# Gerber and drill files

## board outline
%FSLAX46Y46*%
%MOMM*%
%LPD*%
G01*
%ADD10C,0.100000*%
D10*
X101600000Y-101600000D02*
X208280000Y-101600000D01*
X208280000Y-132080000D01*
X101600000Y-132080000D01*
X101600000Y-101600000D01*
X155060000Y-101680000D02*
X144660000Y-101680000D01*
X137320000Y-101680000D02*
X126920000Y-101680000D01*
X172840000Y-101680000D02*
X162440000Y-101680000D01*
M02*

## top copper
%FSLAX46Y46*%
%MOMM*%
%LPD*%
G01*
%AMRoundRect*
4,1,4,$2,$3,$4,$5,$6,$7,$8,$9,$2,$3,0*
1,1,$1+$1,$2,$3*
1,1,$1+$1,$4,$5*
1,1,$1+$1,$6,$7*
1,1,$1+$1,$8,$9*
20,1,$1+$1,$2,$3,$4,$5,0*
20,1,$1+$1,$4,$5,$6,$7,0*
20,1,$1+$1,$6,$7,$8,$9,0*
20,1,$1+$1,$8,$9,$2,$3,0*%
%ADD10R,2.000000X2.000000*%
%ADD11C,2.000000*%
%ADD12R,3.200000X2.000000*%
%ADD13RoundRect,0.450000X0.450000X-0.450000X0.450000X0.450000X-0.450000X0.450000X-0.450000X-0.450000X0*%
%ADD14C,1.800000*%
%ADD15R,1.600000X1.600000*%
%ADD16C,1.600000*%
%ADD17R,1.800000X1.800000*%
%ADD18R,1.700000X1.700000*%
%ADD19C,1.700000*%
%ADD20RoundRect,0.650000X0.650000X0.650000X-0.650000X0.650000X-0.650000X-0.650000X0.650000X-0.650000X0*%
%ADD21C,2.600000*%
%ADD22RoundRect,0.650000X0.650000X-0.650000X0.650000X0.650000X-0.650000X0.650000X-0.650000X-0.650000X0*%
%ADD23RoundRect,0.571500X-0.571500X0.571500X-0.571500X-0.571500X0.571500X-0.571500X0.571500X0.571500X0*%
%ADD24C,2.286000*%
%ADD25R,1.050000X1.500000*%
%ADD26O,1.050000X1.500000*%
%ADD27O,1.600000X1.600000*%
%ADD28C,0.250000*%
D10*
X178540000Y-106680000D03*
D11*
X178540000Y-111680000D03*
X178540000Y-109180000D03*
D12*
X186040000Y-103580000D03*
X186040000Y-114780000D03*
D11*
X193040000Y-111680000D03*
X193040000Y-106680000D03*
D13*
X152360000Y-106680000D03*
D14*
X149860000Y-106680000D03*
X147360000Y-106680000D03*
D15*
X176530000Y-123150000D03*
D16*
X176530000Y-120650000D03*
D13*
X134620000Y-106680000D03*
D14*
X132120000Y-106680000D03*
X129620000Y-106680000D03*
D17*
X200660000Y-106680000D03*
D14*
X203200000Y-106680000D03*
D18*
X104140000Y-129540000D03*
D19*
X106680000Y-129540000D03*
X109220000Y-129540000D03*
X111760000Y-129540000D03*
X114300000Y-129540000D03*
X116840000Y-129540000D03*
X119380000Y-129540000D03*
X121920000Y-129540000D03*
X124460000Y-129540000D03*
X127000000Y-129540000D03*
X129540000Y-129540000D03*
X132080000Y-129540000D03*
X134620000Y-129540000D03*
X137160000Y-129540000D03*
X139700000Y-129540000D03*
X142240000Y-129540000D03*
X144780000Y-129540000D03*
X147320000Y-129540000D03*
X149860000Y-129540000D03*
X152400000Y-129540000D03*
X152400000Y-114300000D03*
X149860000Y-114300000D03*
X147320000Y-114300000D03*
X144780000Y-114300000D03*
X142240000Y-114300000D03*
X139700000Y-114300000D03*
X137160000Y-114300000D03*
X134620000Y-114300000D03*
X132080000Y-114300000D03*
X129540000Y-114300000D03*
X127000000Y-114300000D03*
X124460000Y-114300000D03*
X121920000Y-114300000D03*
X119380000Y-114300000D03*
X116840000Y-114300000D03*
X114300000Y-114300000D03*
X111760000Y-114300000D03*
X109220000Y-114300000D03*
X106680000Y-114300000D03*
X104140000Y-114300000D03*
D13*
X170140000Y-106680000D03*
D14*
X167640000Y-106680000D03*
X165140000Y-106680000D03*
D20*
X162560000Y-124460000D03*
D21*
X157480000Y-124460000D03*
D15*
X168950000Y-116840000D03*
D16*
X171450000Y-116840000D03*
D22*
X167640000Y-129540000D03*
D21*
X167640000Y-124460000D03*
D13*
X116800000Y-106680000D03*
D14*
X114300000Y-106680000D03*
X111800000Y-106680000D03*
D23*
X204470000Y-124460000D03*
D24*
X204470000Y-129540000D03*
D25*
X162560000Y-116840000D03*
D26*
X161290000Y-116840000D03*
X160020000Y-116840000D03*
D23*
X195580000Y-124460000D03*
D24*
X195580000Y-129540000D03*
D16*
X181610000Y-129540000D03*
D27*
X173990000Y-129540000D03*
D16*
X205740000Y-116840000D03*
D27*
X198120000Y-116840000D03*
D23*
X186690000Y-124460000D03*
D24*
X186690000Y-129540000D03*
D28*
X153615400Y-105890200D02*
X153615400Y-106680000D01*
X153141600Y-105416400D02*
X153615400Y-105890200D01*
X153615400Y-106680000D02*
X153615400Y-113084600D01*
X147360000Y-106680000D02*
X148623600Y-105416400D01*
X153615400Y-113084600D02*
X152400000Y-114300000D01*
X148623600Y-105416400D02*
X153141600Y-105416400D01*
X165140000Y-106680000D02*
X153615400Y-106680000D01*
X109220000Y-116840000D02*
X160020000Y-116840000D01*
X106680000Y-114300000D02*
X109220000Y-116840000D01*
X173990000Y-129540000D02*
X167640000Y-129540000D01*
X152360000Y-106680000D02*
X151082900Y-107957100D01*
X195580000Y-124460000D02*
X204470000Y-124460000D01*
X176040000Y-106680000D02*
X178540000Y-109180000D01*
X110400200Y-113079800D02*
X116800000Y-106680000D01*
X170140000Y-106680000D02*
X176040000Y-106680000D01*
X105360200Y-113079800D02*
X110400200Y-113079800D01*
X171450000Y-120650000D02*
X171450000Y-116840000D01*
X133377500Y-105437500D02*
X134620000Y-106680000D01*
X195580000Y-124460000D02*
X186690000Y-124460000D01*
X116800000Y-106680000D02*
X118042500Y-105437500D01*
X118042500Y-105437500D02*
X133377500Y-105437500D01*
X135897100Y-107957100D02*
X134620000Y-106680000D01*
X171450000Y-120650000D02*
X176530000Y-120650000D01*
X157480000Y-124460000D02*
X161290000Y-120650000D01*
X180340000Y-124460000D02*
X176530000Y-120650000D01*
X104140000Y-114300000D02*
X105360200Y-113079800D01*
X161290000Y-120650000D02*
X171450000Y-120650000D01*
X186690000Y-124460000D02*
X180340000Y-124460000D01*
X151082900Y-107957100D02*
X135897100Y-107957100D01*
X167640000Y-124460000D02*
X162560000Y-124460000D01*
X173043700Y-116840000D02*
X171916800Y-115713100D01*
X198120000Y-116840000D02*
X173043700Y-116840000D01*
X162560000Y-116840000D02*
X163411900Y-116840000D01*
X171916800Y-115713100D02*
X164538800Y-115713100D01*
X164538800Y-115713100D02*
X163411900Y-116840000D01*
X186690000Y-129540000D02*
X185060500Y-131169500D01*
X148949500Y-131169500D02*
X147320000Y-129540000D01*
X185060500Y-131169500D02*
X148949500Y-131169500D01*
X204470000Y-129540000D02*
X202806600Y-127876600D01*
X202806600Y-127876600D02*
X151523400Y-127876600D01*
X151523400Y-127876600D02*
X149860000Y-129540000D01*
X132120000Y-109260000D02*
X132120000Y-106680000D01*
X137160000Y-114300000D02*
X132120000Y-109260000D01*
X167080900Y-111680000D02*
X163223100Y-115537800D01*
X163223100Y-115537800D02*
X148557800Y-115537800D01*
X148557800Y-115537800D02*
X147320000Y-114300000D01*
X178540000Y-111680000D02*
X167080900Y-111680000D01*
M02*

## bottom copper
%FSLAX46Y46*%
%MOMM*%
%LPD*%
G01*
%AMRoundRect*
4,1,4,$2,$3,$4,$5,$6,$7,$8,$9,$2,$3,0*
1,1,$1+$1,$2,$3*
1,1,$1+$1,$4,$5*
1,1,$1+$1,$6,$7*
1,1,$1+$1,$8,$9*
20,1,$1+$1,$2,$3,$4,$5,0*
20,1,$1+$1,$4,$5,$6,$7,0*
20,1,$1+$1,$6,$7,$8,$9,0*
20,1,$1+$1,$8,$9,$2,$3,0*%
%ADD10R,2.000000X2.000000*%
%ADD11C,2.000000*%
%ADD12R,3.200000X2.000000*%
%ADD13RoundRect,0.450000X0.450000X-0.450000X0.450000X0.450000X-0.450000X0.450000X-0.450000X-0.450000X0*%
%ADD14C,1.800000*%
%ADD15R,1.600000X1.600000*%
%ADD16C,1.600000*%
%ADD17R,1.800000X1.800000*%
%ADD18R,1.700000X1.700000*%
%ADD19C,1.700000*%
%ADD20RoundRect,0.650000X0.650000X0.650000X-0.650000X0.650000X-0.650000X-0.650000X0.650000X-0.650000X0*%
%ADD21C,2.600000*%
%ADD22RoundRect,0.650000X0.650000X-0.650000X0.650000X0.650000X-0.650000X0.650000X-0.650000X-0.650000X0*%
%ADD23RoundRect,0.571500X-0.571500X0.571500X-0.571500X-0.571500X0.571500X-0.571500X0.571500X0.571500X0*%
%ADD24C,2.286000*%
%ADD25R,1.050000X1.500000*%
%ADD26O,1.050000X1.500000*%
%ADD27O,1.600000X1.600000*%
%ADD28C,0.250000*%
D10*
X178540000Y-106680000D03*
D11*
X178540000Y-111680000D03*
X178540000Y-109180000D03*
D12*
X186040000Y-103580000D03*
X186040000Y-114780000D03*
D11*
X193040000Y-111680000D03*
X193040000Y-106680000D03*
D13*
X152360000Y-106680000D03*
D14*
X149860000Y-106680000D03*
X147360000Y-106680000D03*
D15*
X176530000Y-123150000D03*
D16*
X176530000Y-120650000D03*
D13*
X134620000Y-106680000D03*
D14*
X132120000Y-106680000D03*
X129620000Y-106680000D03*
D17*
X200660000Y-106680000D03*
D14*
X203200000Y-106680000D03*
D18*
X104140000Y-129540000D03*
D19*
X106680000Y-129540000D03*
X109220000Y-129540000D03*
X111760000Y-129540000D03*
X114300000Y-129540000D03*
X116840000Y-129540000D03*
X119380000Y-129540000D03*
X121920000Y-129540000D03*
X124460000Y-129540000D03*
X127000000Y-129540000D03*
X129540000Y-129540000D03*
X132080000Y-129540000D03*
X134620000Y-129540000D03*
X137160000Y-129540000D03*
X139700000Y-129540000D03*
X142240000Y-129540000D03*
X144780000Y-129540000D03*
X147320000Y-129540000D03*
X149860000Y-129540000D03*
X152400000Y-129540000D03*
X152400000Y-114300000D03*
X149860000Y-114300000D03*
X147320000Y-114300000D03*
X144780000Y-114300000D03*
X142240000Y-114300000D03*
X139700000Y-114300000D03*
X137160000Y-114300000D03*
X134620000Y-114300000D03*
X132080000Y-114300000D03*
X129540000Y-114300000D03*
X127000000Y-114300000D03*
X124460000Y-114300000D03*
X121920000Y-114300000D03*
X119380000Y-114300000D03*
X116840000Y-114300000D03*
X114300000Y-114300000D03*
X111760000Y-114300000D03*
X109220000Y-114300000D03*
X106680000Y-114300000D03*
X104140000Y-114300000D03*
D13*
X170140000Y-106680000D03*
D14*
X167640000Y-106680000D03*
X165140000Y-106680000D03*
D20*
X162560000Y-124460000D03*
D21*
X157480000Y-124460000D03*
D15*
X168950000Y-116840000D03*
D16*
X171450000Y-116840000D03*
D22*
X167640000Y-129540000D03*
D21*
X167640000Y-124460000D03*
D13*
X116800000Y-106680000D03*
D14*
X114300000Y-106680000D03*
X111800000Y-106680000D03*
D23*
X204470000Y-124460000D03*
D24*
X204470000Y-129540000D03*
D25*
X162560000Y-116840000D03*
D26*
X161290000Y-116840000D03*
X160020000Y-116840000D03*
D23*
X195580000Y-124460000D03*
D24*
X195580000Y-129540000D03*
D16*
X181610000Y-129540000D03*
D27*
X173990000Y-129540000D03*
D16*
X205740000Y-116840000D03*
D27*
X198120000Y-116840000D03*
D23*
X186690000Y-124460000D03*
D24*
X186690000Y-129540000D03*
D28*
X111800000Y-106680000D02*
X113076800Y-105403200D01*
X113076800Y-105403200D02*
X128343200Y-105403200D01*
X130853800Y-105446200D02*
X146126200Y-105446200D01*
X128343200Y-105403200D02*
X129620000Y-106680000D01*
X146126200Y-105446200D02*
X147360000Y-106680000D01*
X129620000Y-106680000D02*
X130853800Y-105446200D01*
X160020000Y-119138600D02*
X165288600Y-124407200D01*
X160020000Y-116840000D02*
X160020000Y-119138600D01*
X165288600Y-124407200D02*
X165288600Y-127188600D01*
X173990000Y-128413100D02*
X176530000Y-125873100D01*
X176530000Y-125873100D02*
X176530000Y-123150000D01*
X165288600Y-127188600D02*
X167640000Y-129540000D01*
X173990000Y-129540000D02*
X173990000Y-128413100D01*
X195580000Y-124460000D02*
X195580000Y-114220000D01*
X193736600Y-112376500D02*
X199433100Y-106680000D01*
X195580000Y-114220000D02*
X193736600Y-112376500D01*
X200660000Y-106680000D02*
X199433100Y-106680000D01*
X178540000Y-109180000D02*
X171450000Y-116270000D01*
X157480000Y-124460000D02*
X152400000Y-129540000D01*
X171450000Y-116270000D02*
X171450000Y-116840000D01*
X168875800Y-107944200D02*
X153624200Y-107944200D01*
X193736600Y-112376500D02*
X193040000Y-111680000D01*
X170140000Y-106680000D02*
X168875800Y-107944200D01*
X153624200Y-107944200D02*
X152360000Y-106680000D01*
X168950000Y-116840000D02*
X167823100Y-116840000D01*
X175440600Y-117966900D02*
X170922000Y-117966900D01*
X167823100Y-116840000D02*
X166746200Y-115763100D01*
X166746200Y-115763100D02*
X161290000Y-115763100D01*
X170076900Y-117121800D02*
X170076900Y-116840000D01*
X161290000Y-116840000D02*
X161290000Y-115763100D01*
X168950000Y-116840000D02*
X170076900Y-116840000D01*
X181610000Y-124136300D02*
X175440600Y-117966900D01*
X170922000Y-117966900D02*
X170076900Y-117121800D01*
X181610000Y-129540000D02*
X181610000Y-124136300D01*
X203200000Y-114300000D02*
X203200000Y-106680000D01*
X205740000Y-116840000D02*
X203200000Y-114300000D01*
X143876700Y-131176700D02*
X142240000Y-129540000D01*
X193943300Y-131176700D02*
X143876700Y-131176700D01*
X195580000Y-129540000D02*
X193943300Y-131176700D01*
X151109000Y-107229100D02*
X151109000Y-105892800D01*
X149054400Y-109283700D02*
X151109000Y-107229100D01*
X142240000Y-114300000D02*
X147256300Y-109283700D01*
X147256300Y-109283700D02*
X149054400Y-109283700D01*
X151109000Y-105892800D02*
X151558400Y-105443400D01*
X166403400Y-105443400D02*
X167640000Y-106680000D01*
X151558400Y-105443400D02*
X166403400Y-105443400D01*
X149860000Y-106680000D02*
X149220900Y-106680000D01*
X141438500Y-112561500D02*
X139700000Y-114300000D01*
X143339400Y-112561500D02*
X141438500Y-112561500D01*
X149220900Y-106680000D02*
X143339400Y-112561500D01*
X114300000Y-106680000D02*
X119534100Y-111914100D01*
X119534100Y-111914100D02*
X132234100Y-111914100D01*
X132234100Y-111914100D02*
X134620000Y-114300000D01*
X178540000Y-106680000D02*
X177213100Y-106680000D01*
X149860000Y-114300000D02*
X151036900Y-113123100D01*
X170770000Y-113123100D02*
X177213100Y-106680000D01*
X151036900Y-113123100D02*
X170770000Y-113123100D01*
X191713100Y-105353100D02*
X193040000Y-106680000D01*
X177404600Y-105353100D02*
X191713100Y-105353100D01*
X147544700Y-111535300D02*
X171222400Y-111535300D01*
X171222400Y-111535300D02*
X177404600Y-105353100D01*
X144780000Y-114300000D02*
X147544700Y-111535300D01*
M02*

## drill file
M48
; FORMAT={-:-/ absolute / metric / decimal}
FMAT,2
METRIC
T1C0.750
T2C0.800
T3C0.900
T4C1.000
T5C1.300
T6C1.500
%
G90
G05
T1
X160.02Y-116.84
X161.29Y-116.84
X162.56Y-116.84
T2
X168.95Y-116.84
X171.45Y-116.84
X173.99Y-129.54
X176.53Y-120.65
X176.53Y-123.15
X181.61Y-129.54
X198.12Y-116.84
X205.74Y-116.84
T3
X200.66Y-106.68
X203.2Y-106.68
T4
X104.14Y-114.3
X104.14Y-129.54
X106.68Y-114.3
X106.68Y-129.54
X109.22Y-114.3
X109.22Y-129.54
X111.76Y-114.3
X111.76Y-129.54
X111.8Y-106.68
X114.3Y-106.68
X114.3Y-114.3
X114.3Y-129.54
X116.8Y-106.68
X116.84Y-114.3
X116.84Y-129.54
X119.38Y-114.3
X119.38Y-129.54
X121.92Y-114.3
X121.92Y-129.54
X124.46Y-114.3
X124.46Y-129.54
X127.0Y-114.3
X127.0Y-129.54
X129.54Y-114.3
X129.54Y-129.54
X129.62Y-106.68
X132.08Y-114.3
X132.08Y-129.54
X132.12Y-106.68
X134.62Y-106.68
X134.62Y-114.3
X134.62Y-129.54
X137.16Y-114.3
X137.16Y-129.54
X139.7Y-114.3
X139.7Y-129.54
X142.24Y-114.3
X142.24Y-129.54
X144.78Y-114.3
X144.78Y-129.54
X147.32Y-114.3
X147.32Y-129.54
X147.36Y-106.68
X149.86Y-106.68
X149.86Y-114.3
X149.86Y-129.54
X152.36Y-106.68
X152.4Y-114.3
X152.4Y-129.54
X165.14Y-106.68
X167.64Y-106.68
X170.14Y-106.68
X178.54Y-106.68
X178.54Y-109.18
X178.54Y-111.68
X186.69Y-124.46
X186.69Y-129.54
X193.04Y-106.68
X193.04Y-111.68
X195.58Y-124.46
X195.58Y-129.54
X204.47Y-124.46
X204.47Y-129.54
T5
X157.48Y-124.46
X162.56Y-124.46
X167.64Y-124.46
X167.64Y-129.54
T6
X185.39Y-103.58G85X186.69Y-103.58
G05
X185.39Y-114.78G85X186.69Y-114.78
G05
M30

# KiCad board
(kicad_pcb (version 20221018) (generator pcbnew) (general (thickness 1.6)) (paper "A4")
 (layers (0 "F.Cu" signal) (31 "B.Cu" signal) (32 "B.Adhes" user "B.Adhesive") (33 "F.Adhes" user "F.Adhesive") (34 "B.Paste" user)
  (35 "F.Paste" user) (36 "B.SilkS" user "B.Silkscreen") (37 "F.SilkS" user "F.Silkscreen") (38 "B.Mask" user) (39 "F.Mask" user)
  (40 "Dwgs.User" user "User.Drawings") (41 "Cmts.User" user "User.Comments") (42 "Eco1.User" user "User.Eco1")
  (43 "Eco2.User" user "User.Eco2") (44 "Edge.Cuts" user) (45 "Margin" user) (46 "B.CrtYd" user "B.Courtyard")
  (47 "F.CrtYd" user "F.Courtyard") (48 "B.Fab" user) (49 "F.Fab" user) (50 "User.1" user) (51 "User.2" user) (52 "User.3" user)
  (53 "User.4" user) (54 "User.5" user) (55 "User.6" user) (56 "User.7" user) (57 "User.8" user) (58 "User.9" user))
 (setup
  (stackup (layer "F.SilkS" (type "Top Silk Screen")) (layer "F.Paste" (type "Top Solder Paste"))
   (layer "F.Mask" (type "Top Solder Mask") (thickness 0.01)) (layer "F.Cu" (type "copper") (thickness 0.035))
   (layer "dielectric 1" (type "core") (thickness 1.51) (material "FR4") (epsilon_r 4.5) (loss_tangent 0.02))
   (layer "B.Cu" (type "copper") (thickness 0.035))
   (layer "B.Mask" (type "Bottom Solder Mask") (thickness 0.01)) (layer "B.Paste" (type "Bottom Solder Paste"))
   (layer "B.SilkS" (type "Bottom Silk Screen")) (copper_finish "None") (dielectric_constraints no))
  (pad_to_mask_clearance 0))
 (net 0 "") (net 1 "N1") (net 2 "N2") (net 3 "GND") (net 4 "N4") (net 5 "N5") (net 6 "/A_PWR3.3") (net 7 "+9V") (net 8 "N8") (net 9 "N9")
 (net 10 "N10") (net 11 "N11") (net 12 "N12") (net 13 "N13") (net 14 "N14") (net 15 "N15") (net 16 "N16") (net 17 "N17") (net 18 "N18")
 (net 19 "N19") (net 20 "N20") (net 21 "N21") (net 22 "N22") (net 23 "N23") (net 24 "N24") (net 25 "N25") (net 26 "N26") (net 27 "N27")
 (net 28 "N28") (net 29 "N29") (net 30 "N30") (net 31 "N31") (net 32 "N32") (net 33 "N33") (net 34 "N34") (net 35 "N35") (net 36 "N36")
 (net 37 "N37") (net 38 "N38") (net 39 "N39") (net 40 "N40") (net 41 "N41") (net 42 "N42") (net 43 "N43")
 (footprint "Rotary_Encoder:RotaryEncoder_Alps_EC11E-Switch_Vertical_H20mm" (layer "F.Cu") (at 178.54 106.68)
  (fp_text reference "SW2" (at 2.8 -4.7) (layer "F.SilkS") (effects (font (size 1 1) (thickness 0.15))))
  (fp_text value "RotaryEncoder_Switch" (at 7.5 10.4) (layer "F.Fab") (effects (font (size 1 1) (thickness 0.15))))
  (pad "A" thru_hole rect (at 0 0) (size 2 2) (drill 1) (layers "*.Cu" "*.Mask") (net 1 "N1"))
  (pad "B" thru_hole circle (at 0 5) (size 2 2) (drill 1) (layers "*.Cu" "*.Mask") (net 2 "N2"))
  (pad "C" thru_hole circle (at 0 2.5) (size 2 2) (drill 1) (layers "*.Cu" "*.Mask") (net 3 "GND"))
  (pad "MP" thru_hole rect (at 7.5 -3.1) (size 3.2 2) (drill oval 2.8 1.5) (layers "*.Cu" "*.Mask"))
  (pad "MP" thru_hole rect (at 7.5 8.1) (size 3.2 2) (drill oval 2.8 1.5) (layers "*.Cu" "*.Mask"))
  (pad "S1" thru_hole circle (at 14.5 5) (size 2 2) (drill 1) (layers "*.Cu" "*.Mask") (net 3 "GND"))
  (pad "S2" thru_hole circle (at 14.5 0) (size 2 2) (drill 1) (layers "*.Cu" "*.Mask") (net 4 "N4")))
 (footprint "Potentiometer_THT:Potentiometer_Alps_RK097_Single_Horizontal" (layer "F.Cu") (at 152.36 106.68 -90)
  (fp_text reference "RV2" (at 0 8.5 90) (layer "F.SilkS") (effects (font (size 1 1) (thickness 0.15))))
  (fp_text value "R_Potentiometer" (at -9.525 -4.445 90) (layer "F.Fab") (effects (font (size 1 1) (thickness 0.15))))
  (fp_line (start -5 -2.7) (end -5 7.7) (stroke (width 0.1) (type solid)) (layer "Edge.Cuts"))
  (pad "1" thru_hole roundrect (at 0 0 90) (size 1.8 1.8) (drill 1) (layers "*.Cu" "*.Mask") (roundrect_rratio 0.25) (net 3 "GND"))
  (pad "2" thru_hole circle (at 0 2.5 90) (size 1.8 1.8) (drill 1) (layers "*.Cu" "*.Mask") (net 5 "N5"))
  (pad "3" thru_hole circle (at 0 5 90) (size 1.8 1.8) (drill 1) (layers "*.Cu" "*.Mask") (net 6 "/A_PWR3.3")))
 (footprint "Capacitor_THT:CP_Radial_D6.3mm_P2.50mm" (layer "F.Cu") (at 176.53 123.15 90)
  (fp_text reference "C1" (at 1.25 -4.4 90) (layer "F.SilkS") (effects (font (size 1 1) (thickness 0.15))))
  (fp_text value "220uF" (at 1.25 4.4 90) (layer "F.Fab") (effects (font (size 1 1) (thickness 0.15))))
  (pad "1" thru_hole rect (at 0 0 90) (size 1.6 1.6) (drill 0.8) (layers "*.Cu" "*.Mask") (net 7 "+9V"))
  (pad "2" thru_hole circle (at 2.5 0 90) (size 1.6 1.6) (drill 0.8) (layers "*.Cu" "*.Mask") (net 3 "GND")))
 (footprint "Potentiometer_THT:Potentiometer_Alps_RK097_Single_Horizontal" (layer "F.Cu") (at 134.62 106.68 -90)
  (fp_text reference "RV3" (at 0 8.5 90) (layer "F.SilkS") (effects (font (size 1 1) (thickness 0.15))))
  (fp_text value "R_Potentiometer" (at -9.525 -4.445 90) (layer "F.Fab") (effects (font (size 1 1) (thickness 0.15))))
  (fp_line (start -5 -2.7) (end -5 7.7) (stroke (width 0.1) (type solid)) (layer "Edge.Cuts"))
  (pad "1" thru_hole roundrect (at 0 0 90) (size 1.8 1.8) (drill 1) (layers "*.Cu" "*.Mask") (roundrect_rratio 0.25) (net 3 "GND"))
  (pad "2" thru_hole circle (at 0 2.5 90) (size 1.8 1.8) (drill 1) (layers "*.Cu" "*.Mask") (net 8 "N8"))
  (pad "3" thru_hole circle (at 0 5 90) (size 1.8 1.8) (drill 1) (layers "*.Cu" "*.Mask") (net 6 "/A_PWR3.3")))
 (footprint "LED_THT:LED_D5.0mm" (layer "F.Cu") (at 200.66 106.68)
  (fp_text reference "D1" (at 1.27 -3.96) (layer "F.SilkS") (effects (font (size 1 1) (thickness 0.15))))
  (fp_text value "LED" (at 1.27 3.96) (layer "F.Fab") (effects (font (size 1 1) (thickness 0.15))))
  (pad "1" thru_hole rect (at 0 0) (size 1.8 1.8) (drill 0.9) (layers "*.Cu" "*.Mask") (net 3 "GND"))
  (pad "2" thru_hole circle (at 2.54 0) (size 1.8 1.8) (drill 0.9) (layers "*.Cu" "*.Mask") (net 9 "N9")))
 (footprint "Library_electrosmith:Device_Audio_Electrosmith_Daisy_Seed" (layer "F.Cu") (at 104.14 129.54 90)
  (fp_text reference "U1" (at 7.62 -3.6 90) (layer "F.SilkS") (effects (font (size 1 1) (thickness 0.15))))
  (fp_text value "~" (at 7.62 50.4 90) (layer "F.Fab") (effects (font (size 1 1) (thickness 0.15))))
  (pad "1" thru_hole rect (at 0 0 90) (size 1.7 1.7) (drill 1) (layers "*.Cu" "*.Mask") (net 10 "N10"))
  (pad "2" thru_hole circle (at 0 2.54 90) (size 1.7 1.7) (drill 1) (layers "*.Cu" "*.Mask") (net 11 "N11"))
  (pad "3" thru_hole circle (at 0 5.08 90) (size 1.7 1.7) (drill 1) (layers "*.Cu" "*.Mask") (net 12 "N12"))
  (pad "4" thru_hole circle (at 0 7.62 90) (size 1.7 1.7) (drill 1) (layers "*.Cu" "*.Mask") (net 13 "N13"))
  (pad "5" thru_hole circle (at 0 10.16 90) (size 1.7 1.7) (drill 1) (layers "*.Cu" "*.Mask") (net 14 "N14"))
  (pad "6" thru_hole circle (at 0 12.7 90) (size 1.7 1.7) (drill 1) (layers "*.Cu" "*.Mask") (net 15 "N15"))
  (pad "7" thru_hole circle (at 0 15.24 90) (size 1.7 1.7) (drill 1) (layers "*.Cu" "*.Mask") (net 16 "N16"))
  (pad "8" thru_hole circle (at 0 17.78 90) (size 1.7 1.7) (drill 1) (layers "*.Cu" "*.Mask") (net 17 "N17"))
  (pad "9" thru_hole circle (at 0 20.32 90) (size 1.7 1.7) (drill 1) (layers "*.Cu" "*.Mask") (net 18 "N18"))
  (pad "10" thru_hole circle (at 0 22.86 90) (size 1.7 1.7) (drill 1) (layers "*.Cu" "*.Mask") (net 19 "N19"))
  (pad "11" thru_hole circle (at 0 25.4 90) (size 1.7 1.7) (drill 1) (layers "*.Cu" "*.Mask") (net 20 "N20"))
  (pad "12" thru_hole circle (at 0 27.94 90) (size 1.7 1.7) (drill 1) (layers "*.Cu" "*.Mask") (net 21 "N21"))
  (pad "13" thru_hole circle (at 0 30.48 90) (size 1.7 1.7) (drill 1) (layers "*.Cu" "*.Mask") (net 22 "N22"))
  (pad "14" thru_hole circle (at 0 33.02 90) (size 1.7 1.7) (drill 1) (layers "*.Cu" "*.Mask") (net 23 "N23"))
  (pad "15" thru_hole circle (at 0 35.56 90) (size 1.7 1.7) (drill 1) (layers "*.Cu" "*.Mask") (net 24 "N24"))
  (pad "16" thru_hole circle (at 0 38.1 90) (size 1.7 1.7) (drill 1) (layers "*.Cu" "*.Mask") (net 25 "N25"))
  (pad "17" thru_hole circle (at 0 40.64 90) (size 1.7 1.7) (drill 1) (layers "*.Cu" "*.Mask") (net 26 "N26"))
  (pad "18" thru_hole circle (at 0 43.18 90) (size 1.7 1.7) (drill 1) (layers "*.Cu" "*.Mask") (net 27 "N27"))
  (pad "19" thru_hole circle (at 0 45.72 90) (size 1.7 1.7) (drill 1) (layers "*.Cu" "*.Mask") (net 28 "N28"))
  (pad "20" thru_hole circle (at 0 48.26 90) (size 1.7 1.7) (drill 1) (layers "*.Cu" "*.Mask") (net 3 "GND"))
  (pad "21" thru_hole circle (at 15.24 48.26 90) (size 1.7 1.7) (drill 1) (layers "*.Cu" "*.Mask") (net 6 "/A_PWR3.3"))
  (pad "22" thru_hole circle (at 15.24 45.72 90) (size 1.7 1.7) (drill 1) (layers "*.Cu" "*.Mask") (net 1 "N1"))
  (pad "23" thru_hole circle (at 15.24 43.18 90) (size 1.7 1.7) (drill 1) (layers "*.Cu" "*.Mask") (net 2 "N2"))
  (pad "24" thru_hole circle (at 15.24 40.64 90) (size 1.7 1.7) (drill 1) (layers "*.Cu" "*.Mask") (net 4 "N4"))
  (pad "25" thru_hole circle (at 15.24 38.1 90) (size 1.7 1.7) (drill 1) (layers "*.Cu" "*.Mask") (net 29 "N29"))
  (pad "26" thru_hole circle (at 15.24 35.56 90) (size 1.7 1.7) (drill 1) (layers "*.Cu" "*.Mask") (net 5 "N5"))
  (pad "27" thru_hole circle (at 15.24 33.02 90) (size 1.7 1.7) (drill 1) (layers "*.Cu" "*.Mask") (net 8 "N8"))
  (pad "28" thru_hole circle (at 15.24 30.48 90) (size 1.7 1.7) (drill 1) (layers "*.Cu" "*.Mask") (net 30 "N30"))
  (pad "29" thru_hole circle (at 15.24 27.94 90) (size 1.7 1.7) (drill 1) (layers "*.Cu" "*.Mask") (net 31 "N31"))
  (pad "30" thru_hole circle (at 15.24 25.4 90) (size 1.7 1.7) (drill 1) (layers "*.Cu" "*.Mask") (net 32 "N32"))
  (pad "31" thru_hole circle (at 15.24 22.86 90) (size 1.7 1.7) (drill 1) (layers "*.Cu" "*.Mask") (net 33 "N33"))
  (pad "32" thru_hole circle (at 15.24 20.32 90) (size 1.7 1.7) (drill 1) (layers "*.Cu" "*.Mask") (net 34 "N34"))
  (pad "33" thru_hole circle (at 15.24 17.78 90) (size 1.7 1.7) (drill 1) (layers "*.Cu" "*.Mask") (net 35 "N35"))
  (pad "34" thru_hole circle (at 15.24 15.24 90) (size 1.7 1.7) (drill 1) (layers "*.Cu" "*.Mask") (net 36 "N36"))
  (pad "35" thru_hole circle (at 15.24 12.7 90) (size 1.7 1.7) (drill 1) (layers "*.Cu" "*.Mask") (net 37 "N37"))
  (pad "36" thru_hole circle (at 15.24 10.16 90) (size 1.7 1.7) (drill 1) (layers "*.Cu" "*.Mask") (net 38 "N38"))
  (pad "37" thru_hole circle (at 15.24 7.62 90) (size 1.7 1.7) (drill 1) (layers "*.Cu" "*.Mask") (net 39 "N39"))
  (pad "38" thru_hole circle (at 15.24 5.08 90) (size 1.7 1.7) (drill 1) (layers "*.Cu" "*.Mask") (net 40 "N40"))
  (pad "39" thru_hole circle (at 15.24 2.54 90) (size 1.7 1.7) (drill 1) (layers "*.Cu" "*.Mask") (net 7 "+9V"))
  (pad "40" thru_hole circle (at 15.24 0 90) (size 1.7 1.7) (drill 1) (layers "*.Cu" "*.Mask") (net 3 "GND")))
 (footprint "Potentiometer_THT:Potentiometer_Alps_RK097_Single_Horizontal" (layer "F.Cu") (at 170.14 106.68 -90)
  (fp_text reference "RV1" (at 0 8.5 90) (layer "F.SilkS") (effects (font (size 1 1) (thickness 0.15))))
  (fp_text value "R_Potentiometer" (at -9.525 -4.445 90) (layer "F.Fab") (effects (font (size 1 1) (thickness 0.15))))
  (fp_line (start -5 -2.7) (end -5 7.7) (stroke (width 0.1) (type solid)) (layer "Edge.Cuts"))
  (pad "1" thru_hole roundrect (at 0 0 90) (size 1.8 1.8) (drill 1) (layers "*.Cu" "*.Mask") (roundrect_rratio 0.25) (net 3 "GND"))
  (pad "2" thru_hole circle (at 0 2.5 90) (size 1.8 1.8) (drill 1) (layers "*.Cu" "*.Mask") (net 29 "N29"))
  (pad "3" thru_hole circle (at 0 5 90) (size 1.8 1.8) (drill 1) (layers "*.Cu" "*.Mask") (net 6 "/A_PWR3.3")))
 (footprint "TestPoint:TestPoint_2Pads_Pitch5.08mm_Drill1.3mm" (layer "F.Cu") (at 162.56 124.46 180)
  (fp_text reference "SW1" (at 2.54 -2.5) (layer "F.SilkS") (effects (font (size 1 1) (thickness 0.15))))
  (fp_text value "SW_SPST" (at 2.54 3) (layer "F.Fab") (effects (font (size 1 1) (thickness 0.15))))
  (pad "1" thru_hole roundrect (at 0 0 180) (size 2.6 2.6) (drill 1.3) (layers "*.Cu" "*.Mask") (roundrect_rratio 0.25) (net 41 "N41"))
  (pad "2" thru_hole circle (at 5.08 0 180) (size 2.6 2.6) (drill 1.3) (layers "*.Cu" "*.Mask") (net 3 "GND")))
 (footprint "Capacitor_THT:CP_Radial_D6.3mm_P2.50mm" (layer "F.Cu") (at 168.95 116.84)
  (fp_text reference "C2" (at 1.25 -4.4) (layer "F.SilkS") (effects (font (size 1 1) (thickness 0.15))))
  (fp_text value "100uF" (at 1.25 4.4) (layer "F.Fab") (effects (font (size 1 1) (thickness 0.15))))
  (pad "1" thru_hole rect (at 0 0) (size 1.6 1.6) (drill 0.8) (layers "*.Cu" "*.Mask") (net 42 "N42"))
  (pad "2" thru_hole circle (at 2.5 0) (size 1.6 1.6) (drill 0.8) (layers "*.Cu" "*.Mask") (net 3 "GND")))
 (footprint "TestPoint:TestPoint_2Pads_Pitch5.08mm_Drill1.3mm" (layer "F.Cu") (at 167.64 129.54 90)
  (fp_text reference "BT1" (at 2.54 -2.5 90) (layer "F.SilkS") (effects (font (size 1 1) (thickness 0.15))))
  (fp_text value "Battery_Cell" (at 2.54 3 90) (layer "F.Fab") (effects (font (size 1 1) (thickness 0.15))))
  (pad "1" thru_hole roundrect (at 0 0 90) (size 2.6 2.6) (drill 1.3) (layers "*.Cu" "*.Mask") (roundrect_rratio 0.25) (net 7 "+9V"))
  (pad "2" thru_hole circle (at 5.08 0 90) (size 2.6 2.6) (drill 1.3) (layers "*.Cu" "*.Mask") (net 41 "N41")))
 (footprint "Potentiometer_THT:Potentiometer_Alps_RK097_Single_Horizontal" (layer "F.Cu") (at 116.8 106.68 -90)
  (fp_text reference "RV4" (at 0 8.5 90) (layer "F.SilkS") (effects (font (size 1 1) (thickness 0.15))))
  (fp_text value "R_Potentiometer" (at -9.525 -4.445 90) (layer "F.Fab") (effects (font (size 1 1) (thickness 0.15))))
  (pad "1" thru_hole roundrect (at 0 0 90) (size 1.8 1.8) (drill 1) (layers "*.Cu" "*.Mask") (roundrect_rratio 0.25) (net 3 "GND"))
  (pad "2" thru_hole circle (at 0 2.5 90) (size 1.8 1.8) (drill 1) (layers "*.Cu" "*.Mask") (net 30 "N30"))
  (pad "3" thru_hole circle (at 0 5 90) (size 1.8 1.8) (drill 1) (layers "*.Cu" "*.Mask") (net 6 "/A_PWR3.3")))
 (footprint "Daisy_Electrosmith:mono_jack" (layer "F.Cu") (at 204.47 127 -90)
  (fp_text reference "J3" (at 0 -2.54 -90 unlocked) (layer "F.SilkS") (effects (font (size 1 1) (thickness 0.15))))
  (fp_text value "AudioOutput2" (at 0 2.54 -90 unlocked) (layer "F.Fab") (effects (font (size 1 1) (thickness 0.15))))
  (pad "S" thru_hole roundrect (at -2.54 0 270) (size 2.286 2.286) (drill 1) (layers "*.Cu" "*.Mask") (roundrect_rratio 0.25) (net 3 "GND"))
  (pad "T" thru_hole circle (at 2.54 0 270) (size 2.286 2.286) (drill 1) (layers "*.Cu" "*.Mask") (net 28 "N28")))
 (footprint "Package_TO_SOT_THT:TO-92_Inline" (layer "F.Cu") (at 162.56 116.84 180)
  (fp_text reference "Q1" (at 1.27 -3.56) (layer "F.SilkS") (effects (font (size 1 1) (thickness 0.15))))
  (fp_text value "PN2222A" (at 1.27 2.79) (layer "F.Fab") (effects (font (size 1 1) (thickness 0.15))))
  (pad "1" thru_hole rect (at 0 0 180) (size 1.05 1.5) (drill 0.75) (layers "*.Cu" "*.Mask") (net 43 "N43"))
  (pad "2" thru_hole oval (at 1.27 0 180) (size 1.05 1.5) (drill 0.75) (layers "*.Cu" "*.Mask") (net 42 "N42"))
  (pad "3" thru_hole oval (at 2.54 0 180) (size 1.05 1.5) (drill 0.75) (layers "*.Cu" "*.Mask") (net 7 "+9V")))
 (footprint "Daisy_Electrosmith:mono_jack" (layer "F.Cu") (at 195.58 127 -90)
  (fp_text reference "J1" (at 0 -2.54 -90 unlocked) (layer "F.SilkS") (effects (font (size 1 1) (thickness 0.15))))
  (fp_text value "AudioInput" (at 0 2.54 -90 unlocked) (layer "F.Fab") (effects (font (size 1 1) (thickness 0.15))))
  (pad "S" thru_hole roundrect (at -2.54 0 270) (size 2.286 2.286) (drill 1) (layers "*.Cu" "*.Mask") (roundrect_rratio 0.25) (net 3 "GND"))
  (pad "T" thru_hole circle (at 2.54 0 270) (size 2.286 2.286) (drill 1) (layers "*.Cu" "*.Mask") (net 25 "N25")))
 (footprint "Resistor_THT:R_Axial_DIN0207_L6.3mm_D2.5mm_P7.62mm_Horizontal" (layer "F.Cu") (at 181.61 129.54 180)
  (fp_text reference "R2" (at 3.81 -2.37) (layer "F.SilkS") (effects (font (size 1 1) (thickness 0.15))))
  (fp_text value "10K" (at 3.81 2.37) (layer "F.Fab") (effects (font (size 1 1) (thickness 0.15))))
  (pad "1" thru_hole circle (at 0 0 180) (size 1.6 1.6) (drill 0.8) (layers "*.Cu" "*.Mask") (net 42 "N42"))
  (pad "2" thru_hole oval (at 7.62 0 180) (size 1.6 1.6) (drill 0.8) (layers "*.Cu" "*.Mask") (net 7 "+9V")))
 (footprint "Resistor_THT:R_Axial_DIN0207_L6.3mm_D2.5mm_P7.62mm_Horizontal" (layer "F.Cu") (at 205.74 116.84 180)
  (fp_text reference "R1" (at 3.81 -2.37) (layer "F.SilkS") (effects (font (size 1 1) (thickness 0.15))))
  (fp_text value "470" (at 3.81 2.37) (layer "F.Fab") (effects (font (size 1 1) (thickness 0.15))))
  (pad "1" thru_hole circle (at 0 0 180) (size 1.6 1.6) (drill 0.8) (layers "*.Cu" "*.Mask") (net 9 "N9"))
  (pad "2" thru_hole oval (at 7.62 0 180) (size 1.6 1.6) (drill 0.8) (layers "*.Cu" "*.Mask") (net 43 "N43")))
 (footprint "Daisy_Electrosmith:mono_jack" (layer "F.Cu") (at 186.69 127 -90)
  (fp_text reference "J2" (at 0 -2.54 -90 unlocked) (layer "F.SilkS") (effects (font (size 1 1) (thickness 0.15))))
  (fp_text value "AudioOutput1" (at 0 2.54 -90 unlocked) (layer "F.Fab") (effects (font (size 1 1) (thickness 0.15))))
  (pad "S" thru_hole roundrect (at -2.54 0 270) (size 2.286 2.286) (drill 1) (layers "*.Cu" "*.Mask") (roundrect_rratio 0.25) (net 3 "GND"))
  (pad "T" thru_hole circle (at 2.54 0 270) (size 2.286 2.286) (drill 1) (layers "*.Cu" "*.Mask") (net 27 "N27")))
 (gr_rect (start 101.6 101.6) (end 208.28 132.08) (stroke (width 0.1) (type default)) (fill none) (layer "Edge.Cuts"))
 (segment (start 153.6154 105.8902) (end 153.6154 106.68) (width 0.25) (layer "F.Cu") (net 6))
 (segment (start 153.1416 105.4164) (end 153.6154 105.8902) (width 0.25) (layer "F.Cu") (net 6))
 (segment (start 153.6154 106.68) (end 153.6154 113.0846) (width 0.25) (layer "F.Cu") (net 6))
 (segment (start 147.36 106.68) (end 148.6236 105.4164) (width 0.25) (layer "F.Cu") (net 6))
 (segment (start 153.6154 113.0846) (end 152.4 114.3) (width 0.25) (layer "F.Cu") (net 6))
 (segment (start 148.6236 105.4164) (end 153.1416 105.4164) (width 0.25) (layer "F.Cu") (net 6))
 (segment (start 165.14 106.68) (end 153.6154 106.68) (width 0.25) (layer "F.Cu") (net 6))
 (segment (start 111.8 106.68) (end 113.0768 105.4032) (width 0.25) (layer "B.Cu") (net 6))
 (segment (start 113.0768 105.4032) (end 128.3432 105.4032) (width 0.25) (layer "B.Cu") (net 6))
 (segment (start 130.8538 105.4462) (end 146.1262 105.4462) (width 0.25) (layer "B.Cu") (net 6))
 (segment (start 128.3432 105.4032) (end 129.62 106.68) (width 0.25) (layer "B.Cu") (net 6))
 (segment (start 146.1262 105.4462) (end 147.36 106.68) (width 0.25) (layer "B.Cu") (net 6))
 (segment (start 129.62 106.68) (end 130.8538 105.4462) (width 0.25) (layer "B.Cu") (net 6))
 (segment (start 109.22 116.84) (end 160.02 116.84) (width 0.25) (layer "F.Cu") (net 7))
 (segment (start 106.68 114.3) (end 109.22 116.84) (width 0.25) (layer "F.Cu") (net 7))
 (segment (start 173.99 129.54) (end 167.64 129.54) (width 0.25) (layer "F.Cu") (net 7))
 (segment (start 160.02 119.1386) (end 165.2886 124.4072) (width 0.25) (layer "B.Cu") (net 7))
 (segment (start 160.02 116.84) (end 160.02 119.1386) (width 0.25) (layer "B.Cu") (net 7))
 (segment (start 165.2886 124.4072) (end 165.2886 127.1886) (width 0.25) (layer "B.Cu") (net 7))
 (segment (start 173.99 128.4131) (end 176.53 125.8731) (width 0.25) (layer "B.Cu") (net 7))
 (segment (start 176.53 125.8731) (end 176.53 123.15) (width 0.25) (layer "B.Cu") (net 7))
 (segment (start 165.2886 127.1886) (end 167.64 129.54) (width 0.25) (layer "B.Cu") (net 7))
 (segment (start 173.99 129.54) (end 173.99 128.4131) (width 0.25) (layer "B.Cu") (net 7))
 (segment (start 152.36 106.68) (end 151.0829 107.9571) (width 0.25) (layer "F.Cu") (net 3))
 (segment (start 195.58 124.46) (end 204.47 124.46) (width 0.25) (layer "F.Cu") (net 3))
 (segment (start 176.04 106.68) (end 178.54 109.18) (width 0.25) (layer "F.Cu") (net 3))
 (segment (start 110.4002 113.0798) (end 116.8 106.68) (width 0.25) (layer "F.Cu") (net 3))
 (segment (start 170.14 106.68) (end 176.04 106.68) (width 0.25) (layer "F.Cu") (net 3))
 (segment (start 105.3602 113.0798) (end 110.4002 113.0798) (width 0.25) (layer "F.Cu") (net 3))
 (segment (start 171.45 120.65) (end 171.45 116.84) (width 0.25) (layer "F.Cu") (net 3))
 (segment (start 133.3775 105.4375) (end 134.62 106.68) (width 0.25) (layer "F.Cu") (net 3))
 (segment (start 195.58 124.46) (end 186.69 124.46) (width 0.25) (layer "F.Cu") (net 3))
 (segment (start 116.8 106.68) (end 118.0425 105.4375) (width 0.25) (layer "F.Cu") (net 3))
 (segment (start 118.0425 105.4375) (end 133.3775 105.4375) (width 0.25) (layer "F.Cu") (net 3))
 (segment (start 135.8971 107.9571) (end 134.62 106.68) (width 0.25) (layer "F.Cu") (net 3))
 (segment (start 171.45 120.65) (end 176.53 120.65) (width 0.25) (layer "F.Cu") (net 3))
 (segment (start 157.48 124.46) (end 161.29 120.65) (width 0.25) (layer "F.Cu") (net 3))
 (segment (start 180.34 124.46) (end 176.53 120.65) (width 0.25) (layer "F.Cu") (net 3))
 (segment (start 104.14 114.3) (end 105.3602 113.0798) (width 0.25) (layer "F.Cu") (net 3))
 (segment (start 161.29 120.65) (end 171.45 120.65) (width 0.25) (layer "F.Cu") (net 3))
 (segment (start 186.69 124.46) (end 180.34 124.46) (width 0.25) (layer "F.Cu") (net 3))
 (segment (start 151.0829 107.9571) (end 135.8971 107.9571) (width 0.25) (layer "F.Cu") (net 3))
 (segment (start 195.58 124.46) (end 195.58 114.22) (width 0.25) (layer "B.Cu") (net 3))
 (segment (start 193.7366 112.3765) (end 199.4331 106.68) (width 0.25) (layer "B.Cu") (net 3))
 (segment (start 195.58 114.22) (end 193.7366 112.3765) (width 0.25) (layer "B.Cu") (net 3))
 (segment (start 200.66 106.68) (end 199.4331 106.68) (width 0.25) (layer "B.Cu") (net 3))
 (segment (start 178.54 109.18) (end 171.45 116.27) (width 0.25) (layer "B.Cu") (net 3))
 (segment (start 157.48 124.46) (end 152.4 129.54) (width 0.25) (layer "B.Cu") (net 3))
 (segment (start 171.45 116.27) (end 171.45 116.84) (width 0.25) (layer "B.Cu") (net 3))
 (segment (start 168.8758 107.9442) (end 153.6242 107.9442) (width 0.25) (layer "B.Cu") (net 3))
 (segment (start 193.7366 112.3765) (end 193.04 111.68) (width 0.25) (layer "B.Cu") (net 3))
 (segment (start 170.14 106.68) (end 168.8758 107.9442) (width 0.25) (layer "B.Cu") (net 3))
 (segment (start 153.6242 107.9442) (end 152.36 106.68) (width 0.25) (layer "B.Cu") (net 3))
 (segment (start 167.64 124.46) (end 162.56 124.46) (width 0.25) (layer "F.Cu") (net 41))
 (segment (start 168.95 116.84) (end 167.8231 116.84) (width 0.25) (layer "B.Cu") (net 42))
 (segment (start 175.4406 117.9669) (end 170.922 117.9669) (width 0.25) (layer "B.Cu") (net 42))
 (segment (start 167.8231 116.84) (end 166.7462 115.7631) (width 0.25) (layer "B.Cu") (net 42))
 (segment (start 166.7462 115.7631) (end 161.29 115.7631) (width 0.25) (layer "B.Cu") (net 42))
 (segment (start 170.0769 117.1218) (end 170.0769 116.84) (width 0.25) (layer "B.Cu") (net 42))
 (segment (start 161.29 116.84) (end 161.29 115.7631) (width 0.25) (layer "B.Cu") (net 42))
 (segment (start 168.95 116.84) (end 170.0769 116.84) (width 0.25) (layer "B.Cu") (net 42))
 (segment (start 181.61 124.1363) (end 175.4406 117.9669) (width 0.25) (layer "B.Cu") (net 42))
 (segment (start 170.922 117.9669) (end 170.0769 117.1218) (width 0.25) (layer "B.Cu") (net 42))
 (segment (start 181.61 129.54) (end 181.61 124.1363) (width 0.25) (layer "B.Cu") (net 42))
 (segment (start 173.0437 116.84) (end 171.9168 115.7131) (width 0.25) (layer "F.Cu") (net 43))
 (segment (start 198.12 116.84) (end 173.0437 116.84) (width 0.25) (layer "F.Cu") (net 43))
 (segment (start 162.56 116.84) (end 163.4119 116.84) (width 0.25) (layer "F.Cu") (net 43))
 (segment (start 171.9168 115.7131) (end 164.5388 115.7131) (width 0.25) (layer "F.Cu") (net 43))
 (segment (start 164.5388 115.7131) (end 163.4119 116.84) (width 0.25) (layer "F.Cu") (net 43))
 (segment (start 203.2 114.3) (end 203.2 106.68) (width 0.25) (layer "B.Cu") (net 9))
 (segment (start 205.74 116.84) (end 203.2 114.3) (width 0.25) (layer "B.Cu") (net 9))
 (segment (start 143.8767 131.1767) (end 142.24 129.54) (width 0.25) (layer "B.Cu") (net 25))
 (segment (start 193.9433 131.1767) (end 143.8767 131.1767) (width 0.25) (layer "B.Cu") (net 25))
 (segment (start 195.58 129.54) (end 193.9433 131.1767) (width 0.25) (layer "B.Cu") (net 25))
 (segment (start 186.69 129.54) (end 185.0605 131.1695) (width 0.25) (layer "F.Cu") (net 27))
 (segment (start 148.9495 131.1695) (end 147.32 129.54) (width 0.25) (layer "F.Cu") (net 27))
 (segment (start 185.0605 131.1695) (end 148.9495 131.1695) (width 0.25) (layer "F.Cu") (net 27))
 (segment (start 204.47 129.54) (end 202.8066 127.8766) (width 0.25) (layer "F.Cu") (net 28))
 (segment (start 202.8066 127.8766) (end 151.5234 127.8766) (width 0.25) (layer "F.Cu") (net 28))
 (segment (start 151.5234 127.8766) (end 149.86 129.54) (width 0.25) (layer "F.Cu") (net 28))
 (segment (start 151.109 107.2291) (end 151.109 105.8928) (width 0.25) (layer "B.Cu") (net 29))
 (segment (start 149.0544 109.2837) (end 151.109 107.2291) (width 0.25) (layer "B.Cu") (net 29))
 (segment (start 142.24 114.3) (end 147.2563 109.2837) (width 0.25) (layer "B.Cu") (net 29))
 (segment (start 147.2563 109.2837) (end 149.0544 109.2837) (width 0.25) (layer "B.Cu") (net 29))
 (segment (start 151.109 105.8928) (end 151.5584 105.4434) (width 0.25) (layer "B.Cu") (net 29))
 (segment (start 166.4034 105.4434) (end 167.64 106.68) (width 0.25) (layer "B.Cu") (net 29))
 (segment (start 151.5584 105.4434) (end 166.4034 105.4434) (width 0.25) (layer "B.Cu") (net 29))
 (segment (start 149.86 106.68) (end 149.2209 106.68) (width 0.25) (layer "B.Cu") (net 5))
 (segment (start 141.4385 112.5615) (end 139.7 114.3) (width 0.25) (layer "B.Cu") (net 5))
 (segment (start 143.3394 112.5615) (end 141.4385 112.5615) (width 0.25) (layer "B.Cu") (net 5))
 (segment (start 149.2209 106.68) (end 143.3394 112.5615) (width 0.25) (layer "B.Cu") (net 5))
 (segment (start 132.12 109.26) (end 132.12 106.68) (width 0.25) (layer "F.Cu") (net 8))
 (segment (start 137.16 114.3) (end 132.12 109.26) (width 0.25) (layer "F.Cu") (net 8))
 (segment (start 114.3 106.68) (end 119.5341 111.9141) (width 0.25) (layer "B.Cu") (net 30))
 (segment (start 119.5341 111.9141) (end 132.2341 111.9141) (width 0.25) (layer "B.Cu") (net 30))
 (segment (start 132.2341 111.9141) (end 134.62 114.3) (width 0.25) (layer "B.Cu") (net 30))
 (segment (start 178.54 106.68) (end 177.2131 106.68) (width 0.25) (layer "B.Cu") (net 1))
 (segment (start 149.86 114.3) (end 151.0369 113.1231) (width 0.25) (layer "B.Cu") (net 1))
 (segment (start 170.77 113.1231) (end 177.2131 106.68) (width 0.25) (layer "B.Cu") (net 1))
 (segment (start 151.0369 113.1231) (end 170.77 113.1231) (width 0.25) (layer "B.Cu") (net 1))
 (segment (start 167.0809 111.68) (end 163.2231 115.5378) (width 0.25) (layer "F.Cu") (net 2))
 (segment (start 163.2231 115.5378) (end 148.5578 115.5378) (width 0.25) (layer "F.Cu") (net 2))
 (segment (start 148.5578 115.5378) (end 147.32 114.3) (width 0.25) (layer "F.Cu") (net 2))
 (segment (start 178.54 111.68) (end 167.0809 111.68) (width 0.25) (layer "F.Cu") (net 2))
 (segment (start 191.7131 105.3531) (end 193.04 106.68) (width 0.25) (layer "B.Cu") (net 4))
 (segment (start 177.4046 105.3531) (end 191.7131 105.3531) (width 0.25) (layer "B.Cu") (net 4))
 (segment (start 147.5447 111.5353) (end 171.2224 111.5353) (width 0.25) (layer "B.Cu") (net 4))
 (segment (start 171.2224 111.5353) (end 177.4046 105.3531) (width 0.25) (layer "B.Cu") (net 4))
 (segment (start 144.78 114.3) (end 147.5447 111.5353) (width 0.25) (layer "B.Cu") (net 4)))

